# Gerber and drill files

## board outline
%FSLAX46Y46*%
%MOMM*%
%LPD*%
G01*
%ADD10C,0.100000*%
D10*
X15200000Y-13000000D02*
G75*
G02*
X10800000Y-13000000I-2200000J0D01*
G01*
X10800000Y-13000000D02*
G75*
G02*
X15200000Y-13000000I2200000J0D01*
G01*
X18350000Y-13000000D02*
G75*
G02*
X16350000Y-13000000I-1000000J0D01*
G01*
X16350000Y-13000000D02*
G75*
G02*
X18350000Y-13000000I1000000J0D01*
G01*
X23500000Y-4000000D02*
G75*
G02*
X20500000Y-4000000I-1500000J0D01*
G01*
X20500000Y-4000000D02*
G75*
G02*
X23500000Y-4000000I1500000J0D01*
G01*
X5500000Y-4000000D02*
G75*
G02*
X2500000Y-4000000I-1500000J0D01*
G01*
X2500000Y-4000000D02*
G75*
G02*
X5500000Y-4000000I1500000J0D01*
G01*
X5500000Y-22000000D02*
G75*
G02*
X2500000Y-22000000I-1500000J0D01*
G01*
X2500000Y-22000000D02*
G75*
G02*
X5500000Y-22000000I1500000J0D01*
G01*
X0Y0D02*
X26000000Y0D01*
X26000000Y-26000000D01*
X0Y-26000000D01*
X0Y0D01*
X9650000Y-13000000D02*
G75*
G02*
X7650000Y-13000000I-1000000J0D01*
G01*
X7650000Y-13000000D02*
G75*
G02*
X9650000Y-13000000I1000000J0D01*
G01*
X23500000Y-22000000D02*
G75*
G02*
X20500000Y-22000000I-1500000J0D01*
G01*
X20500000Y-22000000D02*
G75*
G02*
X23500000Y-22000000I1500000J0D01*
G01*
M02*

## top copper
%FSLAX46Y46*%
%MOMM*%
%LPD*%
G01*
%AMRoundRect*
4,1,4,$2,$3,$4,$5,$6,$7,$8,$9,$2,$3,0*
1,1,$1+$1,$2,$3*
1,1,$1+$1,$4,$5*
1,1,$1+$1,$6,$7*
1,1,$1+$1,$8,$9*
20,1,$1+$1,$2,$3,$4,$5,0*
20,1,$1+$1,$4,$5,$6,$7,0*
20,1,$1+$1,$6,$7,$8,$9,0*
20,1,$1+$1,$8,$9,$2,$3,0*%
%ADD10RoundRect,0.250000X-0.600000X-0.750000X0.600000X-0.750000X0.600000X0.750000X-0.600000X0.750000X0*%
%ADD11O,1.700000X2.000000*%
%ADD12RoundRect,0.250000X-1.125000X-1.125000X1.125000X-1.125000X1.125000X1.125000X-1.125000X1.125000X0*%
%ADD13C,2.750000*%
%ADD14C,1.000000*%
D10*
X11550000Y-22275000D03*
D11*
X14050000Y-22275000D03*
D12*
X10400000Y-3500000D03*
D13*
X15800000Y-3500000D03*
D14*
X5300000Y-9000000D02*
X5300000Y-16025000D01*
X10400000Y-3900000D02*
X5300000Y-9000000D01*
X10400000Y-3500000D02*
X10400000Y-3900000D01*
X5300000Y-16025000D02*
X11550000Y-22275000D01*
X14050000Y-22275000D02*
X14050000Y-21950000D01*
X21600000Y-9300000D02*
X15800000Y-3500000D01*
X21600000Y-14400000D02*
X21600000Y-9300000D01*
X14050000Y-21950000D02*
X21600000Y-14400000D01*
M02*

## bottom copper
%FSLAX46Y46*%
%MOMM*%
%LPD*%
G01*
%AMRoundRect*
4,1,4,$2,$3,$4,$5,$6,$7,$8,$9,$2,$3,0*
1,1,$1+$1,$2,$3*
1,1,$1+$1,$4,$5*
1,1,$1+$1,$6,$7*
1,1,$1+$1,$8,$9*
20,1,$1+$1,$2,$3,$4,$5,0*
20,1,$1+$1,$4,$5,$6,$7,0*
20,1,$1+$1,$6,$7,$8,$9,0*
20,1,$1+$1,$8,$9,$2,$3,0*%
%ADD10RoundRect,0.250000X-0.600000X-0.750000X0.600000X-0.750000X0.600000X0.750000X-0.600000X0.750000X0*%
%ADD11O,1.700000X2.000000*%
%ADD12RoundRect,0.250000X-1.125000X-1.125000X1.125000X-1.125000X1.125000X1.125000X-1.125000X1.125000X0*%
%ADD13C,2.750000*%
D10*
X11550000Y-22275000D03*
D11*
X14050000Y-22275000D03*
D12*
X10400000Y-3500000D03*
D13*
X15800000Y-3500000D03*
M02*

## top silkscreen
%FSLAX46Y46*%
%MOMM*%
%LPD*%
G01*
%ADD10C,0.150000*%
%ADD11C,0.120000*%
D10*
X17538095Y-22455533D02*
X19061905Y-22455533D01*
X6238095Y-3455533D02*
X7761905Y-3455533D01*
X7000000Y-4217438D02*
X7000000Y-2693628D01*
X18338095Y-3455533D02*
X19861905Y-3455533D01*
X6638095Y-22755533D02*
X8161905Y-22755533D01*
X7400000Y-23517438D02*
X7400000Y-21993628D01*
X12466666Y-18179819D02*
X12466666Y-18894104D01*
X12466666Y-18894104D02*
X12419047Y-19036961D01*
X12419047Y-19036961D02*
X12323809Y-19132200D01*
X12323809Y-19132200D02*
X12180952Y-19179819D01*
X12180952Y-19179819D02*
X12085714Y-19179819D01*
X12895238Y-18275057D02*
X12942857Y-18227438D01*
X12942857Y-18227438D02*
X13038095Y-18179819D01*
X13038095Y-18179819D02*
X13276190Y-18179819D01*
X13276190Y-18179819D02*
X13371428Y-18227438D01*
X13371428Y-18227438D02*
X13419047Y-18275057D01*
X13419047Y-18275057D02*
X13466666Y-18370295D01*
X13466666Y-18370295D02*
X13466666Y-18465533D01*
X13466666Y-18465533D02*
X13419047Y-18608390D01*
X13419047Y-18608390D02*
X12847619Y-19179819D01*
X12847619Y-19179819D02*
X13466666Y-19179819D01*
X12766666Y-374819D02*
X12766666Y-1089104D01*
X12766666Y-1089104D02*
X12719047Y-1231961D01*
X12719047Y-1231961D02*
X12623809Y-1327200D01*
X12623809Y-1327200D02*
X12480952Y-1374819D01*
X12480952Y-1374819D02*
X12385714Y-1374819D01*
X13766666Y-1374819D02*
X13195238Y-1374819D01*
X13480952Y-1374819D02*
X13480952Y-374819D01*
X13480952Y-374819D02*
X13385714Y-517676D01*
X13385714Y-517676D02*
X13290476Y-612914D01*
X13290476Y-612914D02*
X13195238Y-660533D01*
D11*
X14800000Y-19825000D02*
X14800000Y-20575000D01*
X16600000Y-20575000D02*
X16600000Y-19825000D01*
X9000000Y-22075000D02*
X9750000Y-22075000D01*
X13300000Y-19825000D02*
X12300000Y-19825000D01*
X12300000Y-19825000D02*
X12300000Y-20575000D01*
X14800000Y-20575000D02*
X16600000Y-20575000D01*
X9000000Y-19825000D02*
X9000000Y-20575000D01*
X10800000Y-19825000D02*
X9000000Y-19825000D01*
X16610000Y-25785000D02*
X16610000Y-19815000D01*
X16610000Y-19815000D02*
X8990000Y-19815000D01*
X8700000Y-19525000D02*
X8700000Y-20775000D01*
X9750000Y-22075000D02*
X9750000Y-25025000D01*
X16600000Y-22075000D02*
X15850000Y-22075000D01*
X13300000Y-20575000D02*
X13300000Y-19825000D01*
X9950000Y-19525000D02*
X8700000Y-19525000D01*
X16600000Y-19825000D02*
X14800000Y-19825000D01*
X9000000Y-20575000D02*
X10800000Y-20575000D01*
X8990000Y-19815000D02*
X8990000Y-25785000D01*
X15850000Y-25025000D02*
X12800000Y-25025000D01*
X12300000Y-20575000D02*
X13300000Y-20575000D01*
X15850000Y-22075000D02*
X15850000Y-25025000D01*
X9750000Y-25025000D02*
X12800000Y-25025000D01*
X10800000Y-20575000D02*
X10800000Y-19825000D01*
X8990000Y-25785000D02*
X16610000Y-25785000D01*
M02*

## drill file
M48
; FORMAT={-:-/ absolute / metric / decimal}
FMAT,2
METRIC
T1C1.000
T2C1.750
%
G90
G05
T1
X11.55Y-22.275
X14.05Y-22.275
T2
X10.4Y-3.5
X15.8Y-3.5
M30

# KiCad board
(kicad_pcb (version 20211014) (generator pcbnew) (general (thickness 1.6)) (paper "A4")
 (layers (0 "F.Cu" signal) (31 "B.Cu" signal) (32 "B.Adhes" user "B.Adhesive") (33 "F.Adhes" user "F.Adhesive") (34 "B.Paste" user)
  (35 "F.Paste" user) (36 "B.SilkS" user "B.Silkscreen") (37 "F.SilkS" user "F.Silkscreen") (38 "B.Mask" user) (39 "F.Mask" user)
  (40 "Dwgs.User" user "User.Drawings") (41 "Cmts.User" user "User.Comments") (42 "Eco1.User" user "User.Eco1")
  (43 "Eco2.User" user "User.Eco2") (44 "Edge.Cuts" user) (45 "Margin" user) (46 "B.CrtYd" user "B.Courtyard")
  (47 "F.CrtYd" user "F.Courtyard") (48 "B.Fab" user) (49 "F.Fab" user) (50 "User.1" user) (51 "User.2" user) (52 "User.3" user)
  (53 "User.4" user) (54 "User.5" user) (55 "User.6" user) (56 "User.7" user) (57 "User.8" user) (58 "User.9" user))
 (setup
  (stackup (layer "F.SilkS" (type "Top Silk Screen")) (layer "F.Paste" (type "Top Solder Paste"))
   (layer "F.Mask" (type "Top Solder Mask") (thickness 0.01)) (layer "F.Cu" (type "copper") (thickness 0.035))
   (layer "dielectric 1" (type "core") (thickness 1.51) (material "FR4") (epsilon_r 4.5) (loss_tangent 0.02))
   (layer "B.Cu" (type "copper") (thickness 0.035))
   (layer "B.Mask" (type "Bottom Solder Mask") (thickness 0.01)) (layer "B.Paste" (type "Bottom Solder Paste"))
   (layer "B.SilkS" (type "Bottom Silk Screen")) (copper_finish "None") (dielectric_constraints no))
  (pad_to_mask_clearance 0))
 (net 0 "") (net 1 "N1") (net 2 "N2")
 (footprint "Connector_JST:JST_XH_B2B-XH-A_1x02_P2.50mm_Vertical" (layer "F.Cu") (at 11.55 22.275)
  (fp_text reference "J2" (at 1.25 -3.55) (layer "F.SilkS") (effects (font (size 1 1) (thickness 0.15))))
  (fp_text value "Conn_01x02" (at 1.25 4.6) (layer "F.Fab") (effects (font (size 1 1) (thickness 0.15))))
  (fp_line (start 3.25 -2.45) (end 3.25 -1.7) (layer "F.SilkS") (width 0.12))
  (fp_line (start 5.05 -1.7) (end 5.05 -2.45) (layer "F.SilkS") (width 0.12))
  (fp_line (start -2.55 -0.2) (end -1.8 -0.2) (layer "F.SilkS") (width 0.12))
  (fp_line (start 1.75 -2.45) (end 0.75 -2.45) (layer "F.SilkS") (width 0.12))
  (fp_line (start 0.75 -2.45) (end 0.75 -1.7) (layer "F.SilkS") (width 0.12))
  (fp_line (start 3.25 -1.7) (end 5.05 -1.7) (layer "F.SilkS") (width 0.12))
  (fp_line (start -2.55 -2.45) (end -2.55 -1.7) (layer "F.SilkS") (width 0.12))
  (fp_line (start -0.75 -2.45) (end -2.55 -2.45) (layer "F.SilkS") (width 0.12))
  (fp_line (start 5.06 3.51) (end 5.06 -2.46) (layer "F.SilkS") (width 0.12))
  (fp_line (start 5.06 -2.46) (end -2.56 -2.46) (layer "F.SilkS") (width 0.12))
  (fp_line (start -2.85 -2.75) (end -2.85 -1.5) (layer "F.SilkS") (width 0.12))
  (fp_line (start -1.8 -0.2) (end -1.8 2.75) (layer "F.SilkS") (width 0.12))
  (fp_line (start 5.05 -0.2) (end 4.3 -0.2) (layer "F.SilkS") (width 0.12))
  (fp_line (start 1.75 -1.7) (end 1.75 -2.45) (layer "F.SilkS") (width 0.12))
  (fp_line (start -1.6 -2.75) (end -2.85 -2.75) (layer "F.SilkS") (width 0.12))
  (fp_line (start 5.05 -2.45) (end 3.25 -2.45) (layer "F.SilkS") (width 0.12))
  (fp_line (start -2.55 -1.7) (end -0.75 -1.7) (layer "F.SilkS") (width 0.12))
  (fp_line (start -2.56 -2.46) (end -2.56 3.51) (layer "F.SilkS") (width 0.12))
  (fp_line (start 4.3 2.75) (end 1.25 2.75) (layer "F.SilkS") (width 0.12))
  (fp_line (start 0.75 -1.7) (end 1.75 -1.7) (layer "F.SilkS") (width 0.12))
  (fp_line (start 4.3 -0.2) (end 4.3 2.75) (layer "F.SilkS") (width 0.12))
  (fp_line (start -1.8 2.75) (end 1.25 2.75) (layer "F.SilkS") (width 0.12))
  (fp_line (start -0.75 -1.7) (end -0.75 -2.45) (layer "F.SilkS") (width 0.12))
  (fp_line (start -2.56 3.51) (end 5.06 3.51) (layer "F.SilkS") (width 0.12))
  (pad "1" thru_hole roundrect (at 0 0) (size 1.7 2) (drill 1) (layers *.Cu *.Mask) (roundrect_rratio 0.1470588235) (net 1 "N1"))
  (pad "2" thru_hole oval (at 2.5 0) (size 1.7 2) (drill 1) (layers *.Cu *.Mask) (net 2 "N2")))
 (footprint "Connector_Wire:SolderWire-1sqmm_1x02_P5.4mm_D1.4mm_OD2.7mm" (layer "F.Cu") (at 10.4 3.5)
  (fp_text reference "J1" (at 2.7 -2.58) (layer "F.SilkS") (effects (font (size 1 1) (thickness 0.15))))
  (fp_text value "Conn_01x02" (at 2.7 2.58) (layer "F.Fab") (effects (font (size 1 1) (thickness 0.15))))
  (pad "1" thru_hole roundrect (at 0 0) (size 2.75 2.75) (drill 1.75) (layers *.Cu *.Mask) (roundrect_rratio 0.09090909091) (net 1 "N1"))
  (pad "2" thru_hole circle (at 5.4 0) (size 2.75 2.75) (drill 1.75) (layers *.Cu *.Mask) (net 2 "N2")))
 (gr_circle (center 13 13) (end 15.2 13) (layer "Edge.Cuts") (width 0.1) (fill none))
 (gr_circle (center 17.35 13) (end 18.35 13) (layer "Edge.Cuts") (width 0.1) (fill none))
 (gr_circle (center 22 4) (end 23.5 4) (layer "Edge.Cuts") (width 0.1) (fill none))
 (gr_circle (center 4 4) (end 5.5 4) (layer "Edge.Cuts") (width 0.1) (fill none))
 (gr_circle (center 4 22) (end 5.5 22) (layer "Edge.Cuts") (width 0.1) (fill none))
 (gr_rect (start 0 0) (end 26 26) (layer "Edge.Cuts") (width 0.1) (fill none))
 (gr_circle (center 8.65 13) (end 9.65 13) (layer "Edge.Cuts") (width 0.1) (fill none))
 (gr_circle (center 22 22) (end 23.5 22) (layer "Edge.Cuts") (width 0.1) (fill none))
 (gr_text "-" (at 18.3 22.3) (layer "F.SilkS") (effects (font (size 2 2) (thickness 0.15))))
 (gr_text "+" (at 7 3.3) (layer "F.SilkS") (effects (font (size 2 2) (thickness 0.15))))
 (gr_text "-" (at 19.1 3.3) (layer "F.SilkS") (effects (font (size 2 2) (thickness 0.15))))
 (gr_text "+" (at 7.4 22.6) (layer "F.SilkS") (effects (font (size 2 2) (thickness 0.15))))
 (segment (start 5.3 9) (end 5.3 16.025) (width 1) (layer "F.Cu") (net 1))
 (segment (start 10.4 3.9) (end 5.3 9) (width 1) (layer "F.Cu") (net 1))
 (segment (start 10.4 3.5) (end 10.4 3.9) (width 1) (layer "F.Cu") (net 1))
 (segment (start 5.3 16.025) (end 11.55 22.275) (width 1) (layer "F.Cu") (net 1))
 (segment (start 14.05 22.275) (end 14.05 21.95) (width 1) (layer "F.Cu") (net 2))
 (segment (start 21.6 9.3) (end 15.8 3.5) (width 1) (layer "F.Cu") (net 2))
 (segment (start 21.6 14.4) (end 21.6 9.3) (width 1) (layer "F.Cu") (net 2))
 (segment (start 14.05 21.95) (end 21.6 14.4) (width 1) (layer "F.Cu") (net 2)))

